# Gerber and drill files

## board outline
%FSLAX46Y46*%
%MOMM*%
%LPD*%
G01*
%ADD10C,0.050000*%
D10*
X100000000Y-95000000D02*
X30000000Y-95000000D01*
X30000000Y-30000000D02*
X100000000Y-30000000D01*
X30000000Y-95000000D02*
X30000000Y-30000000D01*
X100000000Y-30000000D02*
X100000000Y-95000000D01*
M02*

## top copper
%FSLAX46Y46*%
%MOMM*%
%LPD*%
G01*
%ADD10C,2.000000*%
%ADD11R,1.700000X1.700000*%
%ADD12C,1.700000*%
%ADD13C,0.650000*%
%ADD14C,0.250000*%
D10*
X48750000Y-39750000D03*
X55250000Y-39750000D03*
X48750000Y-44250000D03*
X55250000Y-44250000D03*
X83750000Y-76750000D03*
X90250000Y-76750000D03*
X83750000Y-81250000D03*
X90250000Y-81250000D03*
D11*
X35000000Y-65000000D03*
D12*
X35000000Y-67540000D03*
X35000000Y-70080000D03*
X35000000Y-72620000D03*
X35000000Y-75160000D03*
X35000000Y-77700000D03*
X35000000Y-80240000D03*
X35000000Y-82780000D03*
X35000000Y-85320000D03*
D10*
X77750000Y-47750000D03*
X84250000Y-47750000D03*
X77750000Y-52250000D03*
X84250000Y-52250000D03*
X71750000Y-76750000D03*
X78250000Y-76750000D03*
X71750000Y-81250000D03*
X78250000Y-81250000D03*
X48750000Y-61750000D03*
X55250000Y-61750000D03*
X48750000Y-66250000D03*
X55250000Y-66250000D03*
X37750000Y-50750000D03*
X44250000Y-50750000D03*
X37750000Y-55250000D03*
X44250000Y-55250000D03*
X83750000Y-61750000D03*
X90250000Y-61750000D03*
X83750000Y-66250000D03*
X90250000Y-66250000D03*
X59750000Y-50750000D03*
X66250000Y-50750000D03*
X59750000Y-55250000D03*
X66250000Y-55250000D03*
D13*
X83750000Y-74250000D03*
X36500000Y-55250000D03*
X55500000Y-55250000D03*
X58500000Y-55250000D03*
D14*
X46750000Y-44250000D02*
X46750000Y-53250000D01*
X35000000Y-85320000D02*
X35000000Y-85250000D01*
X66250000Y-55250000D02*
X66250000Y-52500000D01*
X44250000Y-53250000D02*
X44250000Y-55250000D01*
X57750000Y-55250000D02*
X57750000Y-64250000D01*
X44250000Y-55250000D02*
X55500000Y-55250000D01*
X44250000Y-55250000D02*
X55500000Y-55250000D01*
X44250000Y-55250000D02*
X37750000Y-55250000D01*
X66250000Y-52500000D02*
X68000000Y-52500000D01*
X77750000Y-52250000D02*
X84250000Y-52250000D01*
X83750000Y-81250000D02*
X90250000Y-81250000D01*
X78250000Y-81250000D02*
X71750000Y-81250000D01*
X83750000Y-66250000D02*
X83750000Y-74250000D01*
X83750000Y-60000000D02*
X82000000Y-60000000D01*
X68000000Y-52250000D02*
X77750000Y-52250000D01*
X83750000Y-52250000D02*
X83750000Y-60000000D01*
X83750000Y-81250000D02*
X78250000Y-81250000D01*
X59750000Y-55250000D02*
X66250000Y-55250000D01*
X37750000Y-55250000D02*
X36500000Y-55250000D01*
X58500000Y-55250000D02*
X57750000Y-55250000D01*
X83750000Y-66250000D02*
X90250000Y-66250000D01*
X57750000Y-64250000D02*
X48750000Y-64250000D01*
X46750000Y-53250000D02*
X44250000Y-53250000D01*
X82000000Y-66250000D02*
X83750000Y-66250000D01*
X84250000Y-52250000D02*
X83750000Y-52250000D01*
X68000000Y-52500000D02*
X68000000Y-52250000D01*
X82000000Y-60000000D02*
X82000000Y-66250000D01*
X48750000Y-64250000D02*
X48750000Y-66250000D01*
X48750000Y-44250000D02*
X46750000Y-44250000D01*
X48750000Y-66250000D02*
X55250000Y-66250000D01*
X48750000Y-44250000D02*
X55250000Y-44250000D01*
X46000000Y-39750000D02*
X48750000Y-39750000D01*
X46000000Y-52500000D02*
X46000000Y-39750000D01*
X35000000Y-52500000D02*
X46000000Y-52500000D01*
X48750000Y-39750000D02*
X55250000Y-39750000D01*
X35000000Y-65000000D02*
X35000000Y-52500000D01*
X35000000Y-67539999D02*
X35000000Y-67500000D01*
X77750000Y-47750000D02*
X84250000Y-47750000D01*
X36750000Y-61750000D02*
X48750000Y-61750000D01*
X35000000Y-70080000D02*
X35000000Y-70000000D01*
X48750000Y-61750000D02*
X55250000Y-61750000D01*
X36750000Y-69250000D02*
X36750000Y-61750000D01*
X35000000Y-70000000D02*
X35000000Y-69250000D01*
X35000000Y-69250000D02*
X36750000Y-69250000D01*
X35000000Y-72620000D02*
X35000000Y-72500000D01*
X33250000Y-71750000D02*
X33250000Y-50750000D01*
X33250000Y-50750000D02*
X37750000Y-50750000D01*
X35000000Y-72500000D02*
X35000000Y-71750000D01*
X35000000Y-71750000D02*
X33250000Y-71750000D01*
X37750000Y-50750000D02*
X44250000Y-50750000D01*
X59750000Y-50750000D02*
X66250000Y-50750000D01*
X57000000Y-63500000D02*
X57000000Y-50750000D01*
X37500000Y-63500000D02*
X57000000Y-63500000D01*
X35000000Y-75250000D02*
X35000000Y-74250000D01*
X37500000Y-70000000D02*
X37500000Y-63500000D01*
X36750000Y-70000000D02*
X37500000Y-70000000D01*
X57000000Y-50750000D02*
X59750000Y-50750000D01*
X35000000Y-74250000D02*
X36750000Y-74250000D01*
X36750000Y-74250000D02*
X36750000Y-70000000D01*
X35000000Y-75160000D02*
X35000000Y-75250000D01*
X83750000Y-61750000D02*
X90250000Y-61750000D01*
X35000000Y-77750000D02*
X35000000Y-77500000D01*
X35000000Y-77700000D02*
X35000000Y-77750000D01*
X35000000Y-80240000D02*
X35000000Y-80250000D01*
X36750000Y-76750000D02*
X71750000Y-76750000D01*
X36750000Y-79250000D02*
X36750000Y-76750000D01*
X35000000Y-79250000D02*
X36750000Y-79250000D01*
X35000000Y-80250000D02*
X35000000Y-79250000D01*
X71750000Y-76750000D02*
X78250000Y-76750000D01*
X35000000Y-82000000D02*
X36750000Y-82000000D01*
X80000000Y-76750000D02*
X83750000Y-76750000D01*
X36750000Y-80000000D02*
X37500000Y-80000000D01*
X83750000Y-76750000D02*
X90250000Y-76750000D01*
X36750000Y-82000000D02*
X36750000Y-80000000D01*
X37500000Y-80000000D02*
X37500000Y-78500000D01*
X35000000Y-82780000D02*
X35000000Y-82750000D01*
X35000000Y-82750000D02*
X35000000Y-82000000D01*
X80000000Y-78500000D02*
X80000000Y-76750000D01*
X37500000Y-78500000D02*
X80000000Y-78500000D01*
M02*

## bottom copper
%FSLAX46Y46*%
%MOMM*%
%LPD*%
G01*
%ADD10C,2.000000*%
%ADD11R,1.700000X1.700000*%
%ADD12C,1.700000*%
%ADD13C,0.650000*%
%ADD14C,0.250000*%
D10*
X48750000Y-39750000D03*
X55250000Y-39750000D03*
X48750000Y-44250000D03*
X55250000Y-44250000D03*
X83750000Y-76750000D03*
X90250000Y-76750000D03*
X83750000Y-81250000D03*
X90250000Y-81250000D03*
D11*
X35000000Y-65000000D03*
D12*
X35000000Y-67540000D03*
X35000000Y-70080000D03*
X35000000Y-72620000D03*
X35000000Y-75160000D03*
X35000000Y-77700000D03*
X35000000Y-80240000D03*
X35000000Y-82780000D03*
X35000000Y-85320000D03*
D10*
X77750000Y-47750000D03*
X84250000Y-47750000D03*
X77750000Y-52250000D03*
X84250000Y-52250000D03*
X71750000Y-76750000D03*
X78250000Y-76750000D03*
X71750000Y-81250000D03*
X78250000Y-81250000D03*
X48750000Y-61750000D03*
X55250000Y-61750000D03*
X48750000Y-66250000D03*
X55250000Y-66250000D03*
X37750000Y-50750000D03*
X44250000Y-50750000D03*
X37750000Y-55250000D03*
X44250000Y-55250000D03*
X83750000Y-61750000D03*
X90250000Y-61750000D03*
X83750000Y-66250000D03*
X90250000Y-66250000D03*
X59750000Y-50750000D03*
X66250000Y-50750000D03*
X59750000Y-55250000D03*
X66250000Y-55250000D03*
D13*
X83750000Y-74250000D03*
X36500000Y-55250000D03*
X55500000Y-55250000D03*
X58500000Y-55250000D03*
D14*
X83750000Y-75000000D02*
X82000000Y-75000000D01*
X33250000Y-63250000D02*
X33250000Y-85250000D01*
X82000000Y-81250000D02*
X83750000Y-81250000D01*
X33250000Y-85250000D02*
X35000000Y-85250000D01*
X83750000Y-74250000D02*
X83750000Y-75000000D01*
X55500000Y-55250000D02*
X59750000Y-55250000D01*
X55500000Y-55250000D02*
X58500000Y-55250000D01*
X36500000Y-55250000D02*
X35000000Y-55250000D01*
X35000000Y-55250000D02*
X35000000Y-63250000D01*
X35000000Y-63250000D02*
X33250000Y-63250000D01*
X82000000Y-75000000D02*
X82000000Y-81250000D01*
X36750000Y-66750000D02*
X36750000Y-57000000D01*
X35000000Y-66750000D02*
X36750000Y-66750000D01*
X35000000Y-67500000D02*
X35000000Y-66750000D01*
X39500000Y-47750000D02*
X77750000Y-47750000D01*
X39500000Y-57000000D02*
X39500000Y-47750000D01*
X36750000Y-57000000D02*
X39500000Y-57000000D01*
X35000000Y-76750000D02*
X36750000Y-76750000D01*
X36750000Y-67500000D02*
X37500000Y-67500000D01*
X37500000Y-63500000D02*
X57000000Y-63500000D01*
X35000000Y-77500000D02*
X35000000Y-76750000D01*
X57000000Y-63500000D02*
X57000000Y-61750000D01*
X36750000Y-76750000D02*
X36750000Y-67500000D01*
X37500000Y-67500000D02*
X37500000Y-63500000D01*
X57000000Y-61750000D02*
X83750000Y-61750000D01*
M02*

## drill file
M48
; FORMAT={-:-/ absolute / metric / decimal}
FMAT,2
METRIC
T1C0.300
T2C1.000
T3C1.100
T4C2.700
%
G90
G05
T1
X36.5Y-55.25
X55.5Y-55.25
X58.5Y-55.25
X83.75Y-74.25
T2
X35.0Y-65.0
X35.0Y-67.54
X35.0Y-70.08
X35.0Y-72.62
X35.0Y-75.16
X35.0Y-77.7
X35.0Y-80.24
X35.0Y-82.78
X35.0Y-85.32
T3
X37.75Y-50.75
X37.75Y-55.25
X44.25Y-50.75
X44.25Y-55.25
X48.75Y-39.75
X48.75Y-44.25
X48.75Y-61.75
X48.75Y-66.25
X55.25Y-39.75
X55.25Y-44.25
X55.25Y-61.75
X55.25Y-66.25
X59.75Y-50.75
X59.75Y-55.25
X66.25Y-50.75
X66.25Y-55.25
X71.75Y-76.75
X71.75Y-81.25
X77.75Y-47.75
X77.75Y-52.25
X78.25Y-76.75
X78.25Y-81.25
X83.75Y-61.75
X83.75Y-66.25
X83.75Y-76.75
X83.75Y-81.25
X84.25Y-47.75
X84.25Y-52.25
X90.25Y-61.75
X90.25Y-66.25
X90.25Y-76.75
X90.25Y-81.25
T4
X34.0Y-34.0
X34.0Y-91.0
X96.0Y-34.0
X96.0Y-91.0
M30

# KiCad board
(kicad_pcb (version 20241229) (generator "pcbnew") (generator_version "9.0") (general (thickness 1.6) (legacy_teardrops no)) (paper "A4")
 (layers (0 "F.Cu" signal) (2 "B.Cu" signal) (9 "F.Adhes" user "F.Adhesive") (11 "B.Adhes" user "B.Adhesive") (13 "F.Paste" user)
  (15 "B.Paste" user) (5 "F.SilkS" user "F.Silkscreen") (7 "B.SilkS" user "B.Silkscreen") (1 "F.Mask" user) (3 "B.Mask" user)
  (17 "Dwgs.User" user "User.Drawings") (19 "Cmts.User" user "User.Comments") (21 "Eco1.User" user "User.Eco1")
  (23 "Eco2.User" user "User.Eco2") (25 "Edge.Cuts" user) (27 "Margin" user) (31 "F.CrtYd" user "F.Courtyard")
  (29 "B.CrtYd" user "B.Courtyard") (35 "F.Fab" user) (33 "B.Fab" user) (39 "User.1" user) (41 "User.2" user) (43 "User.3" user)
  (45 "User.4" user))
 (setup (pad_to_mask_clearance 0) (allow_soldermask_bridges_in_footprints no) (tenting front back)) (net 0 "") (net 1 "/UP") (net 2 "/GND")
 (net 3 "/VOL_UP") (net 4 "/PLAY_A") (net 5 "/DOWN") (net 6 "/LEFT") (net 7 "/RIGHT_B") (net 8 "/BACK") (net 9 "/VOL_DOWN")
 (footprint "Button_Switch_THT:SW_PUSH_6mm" (layer "F.Cu") (at 48.75 39.75)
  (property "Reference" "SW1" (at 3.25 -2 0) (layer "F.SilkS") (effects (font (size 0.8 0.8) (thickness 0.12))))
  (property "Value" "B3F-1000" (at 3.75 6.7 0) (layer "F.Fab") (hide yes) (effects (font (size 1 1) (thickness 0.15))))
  (pad "1" thru_hole circle (at 0 0 90) (size 2 2) (drill 1.1) (layers "*.Cu" "*.Mask") (remove_unused_layers no) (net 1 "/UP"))
  (pad "1" thru_hole circle (at 6.5 0 90) (size 2 2) (drill 1.1) (layers "*.Cu" "*.Mask") (remove_unused_layers no) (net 1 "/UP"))
  (pad "2" thru_hole circle (at 0 4.5 90) (size 2 2) (drill 1.1) (layers "*.Cu" "*.Mask") (remove_unused_layers no) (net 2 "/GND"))
  (pad "2" thru_hole circle (at 6.5 4.5 90) (size 2 2) (drill 1.1) (layers "*.Cu" "*.Mask") (remove_unused_layers no) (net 2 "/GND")))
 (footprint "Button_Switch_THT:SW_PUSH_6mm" (layer "F.Cu") (at 83.75 76.75)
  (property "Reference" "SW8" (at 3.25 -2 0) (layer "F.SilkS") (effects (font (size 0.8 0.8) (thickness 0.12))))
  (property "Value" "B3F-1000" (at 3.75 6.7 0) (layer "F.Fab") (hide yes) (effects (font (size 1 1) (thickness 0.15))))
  (pad "1" thru_hole circle (at 0 0 90) (size 2 2) (drill 1.1) (layers "*.Cu" "*.Mask") (remove_unused_layers no) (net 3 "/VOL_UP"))
  (pad "1" thru_hole circle (at 6.5 0 90) (size 2 2) (drill 1.1) (layers "*.Cu" "*.Mask") (remove_unused_layers no) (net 3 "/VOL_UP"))
  (pad "2" thru_hole circle (at 0 4.5 90) (size 2 2) (drill 1.1) (layers "*.Cu" "*.Mask") (remove_unused_layers no) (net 2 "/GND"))
  (pad "2" thru_hole circle (at 6.5 4.5 90) (size 2 2) (drill 1.1) (layers "*.Cu" "*.Mask") (remove_unused_layers no) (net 2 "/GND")))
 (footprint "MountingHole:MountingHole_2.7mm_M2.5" (layer "F.Cu") (at 34 91)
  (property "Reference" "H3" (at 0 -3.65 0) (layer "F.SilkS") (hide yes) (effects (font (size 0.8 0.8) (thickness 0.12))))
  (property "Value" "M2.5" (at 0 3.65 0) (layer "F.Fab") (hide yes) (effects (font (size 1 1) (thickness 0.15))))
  (pad "" np_thru_hole circle (at 0 0) (size 2.7 2.7) (drill 2.7) (layers "*.Cu" "*.Mask")))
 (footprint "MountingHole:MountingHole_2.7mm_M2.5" (layer "F.Cu") (at 96 91)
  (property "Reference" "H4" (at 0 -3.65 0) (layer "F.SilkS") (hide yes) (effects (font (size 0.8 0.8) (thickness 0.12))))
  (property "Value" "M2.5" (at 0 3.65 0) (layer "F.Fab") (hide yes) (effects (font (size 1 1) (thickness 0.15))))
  (pad "" np_thru_hole circle (at 0 0) (size 2.7 2.7) (drill 2.7) (layers "*.Cu" "*.Mask")))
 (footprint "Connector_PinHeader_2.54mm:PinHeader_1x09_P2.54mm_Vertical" (layer "F.Cu") (at 35 65)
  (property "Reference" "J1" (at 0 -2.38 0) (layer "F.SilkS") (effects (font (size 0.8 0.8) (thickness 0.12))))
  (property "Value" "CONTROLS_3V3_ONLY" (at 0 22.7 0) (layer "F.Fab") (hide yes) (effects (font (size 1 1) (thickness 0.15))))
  (pad "1" thru_hole rect (at 0 0) (size 1.7 1.7) (drill 1) (layers "*.Cu" "*.Mask") (remove_unused_layers no) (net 1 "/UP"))
  (pad "2" thru_hole circle (at 0 2.54) (size 1.7 1.7) (drill 1) (layers "*.Cu" "*.Mask") (remove_unused_layers no) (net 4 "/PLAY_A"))
  (pad "3" thru_hole circle (at 0 5.08) (size 1.7 1.7) (drill 1) (layers "*.Cu" "*.Mask") (remove_unused_layers no) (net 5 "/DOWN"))
  (pad "4" thru_hole circle (at 0 7.62) (size 1.7 1.7) (drill 1) (layers "*.Cu" "*.Mask") (remove_unused_layers no) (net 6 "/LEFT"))
  (pad "5" thru_hole circle (at 0 10.16) (size 1.7 1.7) (drill 1) (layers "*.Cu" "*.Mask") (remove_unused_layers no) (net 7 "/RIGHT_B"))
  (pad "6" thru_hole circle (at 0 12.7) (size 1.7 1.7) (drill 1) (layers "*.Cu" "*.Mask") (remove_unused_layers no) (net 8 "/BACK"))
  (pad "7" thru_hole circle (at 0 15.24) (size 1.7 1.7) (drill 1) (layers "*.Cu" "*.Mask") (remove_unused_layers no) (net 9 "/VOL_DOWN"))
  (pad "8" thru_hole circle (at 0 17.78) (size 1.7 1.7) (drill 1) (layers "*.Cu" "*.Mask") (remove_unused_layers no) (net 3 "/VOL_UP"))
  (pad "9" thru_hole circle (at 0 20.32) (size 1.7 1.7) (drill 1) (layers "*.Cu" "*.Mask") (remove_unused_layers no) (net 2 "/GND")))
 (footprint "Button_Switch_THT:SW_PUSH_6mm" (layer "F.Cu") (at 77.75 47.75)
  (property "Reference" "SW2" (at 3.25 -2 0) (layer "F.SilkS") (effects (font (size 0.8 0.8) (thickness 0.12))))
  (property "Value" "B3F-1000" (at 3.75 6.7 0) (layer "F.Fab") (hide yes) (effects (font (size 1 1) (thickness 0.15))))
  (pad "1" thru_hole circle (at 0 0 90) (size 2 2) (drill 1.1) (layers "*.Cu" "*.Mask") (remove_unused_layers no) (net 4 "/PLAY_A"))
  (pad "1" thru_hole circle (at 6.5 0 90) (size 2 2) (drill 1.1) (layers "*.Cu" "*.Mask") (remove_unused_layers no) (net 4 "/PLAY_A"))
  (pad "2" thru_hole circle (at 0 4.5 90) (size 2 2) (drill 1.1) (layers "*.Cu" "*.Mask") (remove_unused_layers no) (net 2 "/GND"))
  (pad "2" thru_hole circle (at 6.5 4.5 90) (size 2 2) (drill 1.1) (layers "*.Cu" "*.Mask") (remove_unused_layers no) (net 2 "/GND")))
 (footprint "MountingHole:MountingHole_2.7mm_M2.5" (layer "F.Cu") (at 34 34)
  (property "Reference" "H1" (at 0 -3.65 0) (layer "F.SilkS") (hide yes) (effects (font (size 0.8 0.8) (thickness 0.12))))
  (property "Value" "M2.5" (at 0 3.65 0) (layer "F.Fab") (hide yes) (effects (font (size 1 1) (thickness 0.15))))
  (pad "" np_thru_hole circle (at 0 0) (size 2.7 2.7) (drill 2.7) (layers "*.Cu" "*.Mask")))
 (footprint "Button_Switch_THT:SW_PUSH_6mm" (layer "F.Cu") (at 71.75 76.75)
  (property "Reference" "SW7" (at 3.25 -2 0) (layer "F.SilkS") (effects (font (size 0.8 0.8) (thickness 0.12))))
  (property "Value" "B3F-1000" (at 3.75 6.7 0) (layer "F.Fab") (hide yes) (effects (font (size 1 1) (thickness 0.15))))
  (pad "1" thru_hole circle (at 0 0 90) (size 2 2) (drill 1.1) (layers "*.Cu" "*.Mask") (remove_unused_layers no) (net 9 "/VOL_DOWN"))
  (pad "1" thru_hole circle (at 6.5 0 90) (size 2 2) (drill 1.1) (layers "*.Cu" "*.Mask") (remove_unused_layers no) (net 9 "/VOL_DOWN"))
  (pad "2" thru_hole circle (at 0 4.5 90) (size 2 2) (drill 1.1) (layers "*.Cu" "*.Mask") (remove_unused_layers no) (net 2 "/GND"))
  (pad "2" thru_hole circle (at 6.5 4.5 90) (size 2 2) (drill 1.1) (layers "*.Cu" "*.Mask") (remove_unused_layers no) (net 2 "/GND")))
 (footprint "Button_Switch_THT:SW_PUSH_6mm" (layer "F.Cu") (at 48.75 61.75)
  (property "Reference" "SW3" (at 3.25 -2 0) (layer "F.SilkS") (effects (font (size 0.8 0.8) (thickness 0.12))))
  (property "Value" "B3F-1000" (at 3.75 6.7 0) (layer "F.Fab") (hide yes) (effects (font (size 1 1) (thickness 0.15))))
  (pad "1" thru_hole circle (at 0 0 90) (size 2 2) (drill 1.1) (layers "*.Cu" "*.Mask") (remove_unused_layers no) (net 5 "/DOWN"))
  (pad "1" thru_hole circle (at 6.5 0 90) (size 2 2) (drill 1.1) (layers "*.Cu" "*.Mask") (remove_unused_layers no) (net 5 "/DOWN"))
  (pad "2" thru_hole circle (at 0 4.5 90) (size 2 2) (drill 1.1) (layers "*.Cu" "*.Mask") (remove_unused_layers no) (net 2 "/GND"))
  (pad "2" thru_hole circle (at 6.5 4.5 90) (size 2 2) (drill 1.1) (layers "*.Cu" "*.Mask") (remove_unused_layers no) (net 2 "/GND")))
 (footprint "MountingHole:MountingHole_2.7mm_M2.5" (layer "F.Cu") (at 96 34)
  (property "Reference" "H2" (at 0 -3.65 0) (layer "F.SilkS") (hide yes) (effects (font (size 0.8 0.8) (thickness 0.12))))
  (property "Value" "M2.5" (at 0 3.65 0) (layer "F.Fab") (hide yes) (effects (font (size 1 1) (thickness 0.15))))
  (pad "" np_thru_hole circle (at 0 0) (size 2.7 2.7) (drill 2.7) (layers "*.Cu" "*.Mask")))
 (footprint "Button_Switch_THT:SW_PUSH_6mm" (layer "F.Cu") (at 37.75 50.75)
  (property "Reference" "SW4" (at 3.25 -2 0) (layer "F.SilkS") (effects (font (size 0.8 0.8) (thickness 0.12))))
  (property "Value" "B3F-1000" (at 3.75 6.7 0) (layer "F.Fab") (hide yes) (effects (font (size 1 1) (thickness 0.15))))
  (pad "1" thru_hole circle (at 0 0 90) (size 2 2) (drill 1.1) (layers "*.Cu" "*.Mask") (remove_unused_layers no) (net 6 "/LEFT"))
  (pad "1" thru_hole circle (at 6.5 0 90) (size 2 2) (drill 1.1) (layers "*.Cu" "*.Mask") (remove_unused_layers no) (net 6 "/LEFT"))
  (pad "2" thru_hole circle (at 0 4.5 90) (size 2 2) (drill 1.1) (layers "*.Cu" "*.Mask") (remove_unused_layers no) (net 2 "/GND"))
  (pad "2" thru_hole circle (at 6.5 4.5 90) (size 2 2) (drill 1.1) (layers "*.Cu" "*.Mask") (remove_unused_layers no) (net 2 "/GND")))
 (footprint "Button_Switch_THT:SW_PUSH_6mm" (layer "F.Cu") (at 83.75 61.75)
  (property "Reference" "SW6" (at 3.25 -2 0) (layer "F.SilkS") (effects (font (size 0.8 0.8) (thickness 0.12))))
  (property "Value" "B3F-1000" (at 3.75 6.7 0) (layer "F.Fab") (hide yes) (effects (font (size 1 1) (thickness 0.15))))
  (pad "1" thru_hole circle (at 0 0 90) (size 2 2) (drill 1.1) (layers "*.Cu" "*.Mask") (remove_unused_layers no) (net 8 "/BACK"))
  (pad "1" thru_hole circle (at 6.5 0 90) (size 2 2) (drill 1.1) (layers "*.Cu" "*.Mask") (remove_unused_layers no) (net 8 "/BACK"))
  (pad "2" thru_hole circle (at 0 4.5 90) (size 2 2) (drill 1.1) (layers "*.Cu" "*.Mask") (remove_unused_layers no) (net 2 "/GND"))
  (pad "2" thru_hole circle (at 6.5 4.5 90) (size 2 2) (drill 1.1) (layers "*.Cu" "*.Mask") (remove_unused_layers no) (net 2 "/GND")))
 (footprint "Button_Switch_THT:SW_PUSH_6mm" (layer "F.Cu") (at 59.75 50.75)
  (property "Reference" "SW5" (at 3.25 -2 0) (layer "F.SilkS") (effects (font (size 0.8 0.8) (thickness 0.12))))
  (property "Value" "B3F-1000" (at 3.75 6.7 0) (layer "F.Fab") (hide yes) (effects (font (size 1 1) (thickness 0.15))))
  (pad "1" thru_hole circle (at 0 0 90) (size 2 2) (drill 1.1) (layers "*.Cu" "*.Mask") (remove_unused_layers no) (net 7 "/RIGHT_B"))
  (pad "1" thru_hole circle (at 6.5 0 90) (size 2 2) (drill 1.1) (layers "*.Cu" "*.Mask") (remove_unused_layers no) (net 7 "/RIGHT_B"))
  (pad "2" thru_hole circle (at 0 4.5 90) (size 2 2) (drill 1.1) (layers "*.Cu" "*.Mask") (remove_unused_layers no) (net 2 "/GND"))
  (pad "2" thru_hole circle (at 6.5 4.5 90) (size 2 2) (drill 1.1) (layers "*.Cu" "*.Mask") (remove_unused_layers no) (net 2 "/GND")))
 (gr_line (start 100 95) (end 30 95) (stroke (width 0.05) (type default)) (layer "Edge.Cuts"))
 (gr_line (start 30 30) (end 100 30) (stroke (width 0.05) (type default)) (layer "Edge.Cuts"))
 (gr_line (start 30 95) (end 30 30) (stroke (width 0.05) (type default)) (layer "Edge.Cuts"))
 (gr_line (start 100 30) (end 100 95) (stroke (width 0.05) (type default)) (layer "Edge.Cuts"))
 (segment (start 46.75 44.25) (end 46.75 53.25) (width 0.25) (layer "F.Cu") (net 2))
 (segment (start 35 85.32) (end 35 85.25) (width 0.25) (layer "F.Cu") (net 2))
 (segment (start 66.25 55.25) (end 66.25 52.5) (width 0.25) (layer "F.Cu") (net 2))
 (segment (start 44.25 53.25) (end 44.25 55.25) (width 0.25) (layer "F.Cu") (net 2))
 (segment (start 57.75 55.25) (end 57.75 64.25) (width 0.25) (layer "F.Cu") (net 2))
 (segment (start 44.25 55.25) (end 55.5 55.25) (width 0.25) (layer "F.Cu") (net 2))
 (segment (start 44.25 55.25) (end 55.5 55.25) (width 0.25) (layer "F.Cu") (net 2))
 (segment (start 44.25 55.25) (end 37.75 55.25) (width 0.25) (layer "F.Cu") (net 2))
 (segment (start 66.25 52.5) (end 68 52.5) (width 0.25) (layer "F.Cu") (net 2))
 (segment (start 77.75 52.25) (end 84.25 52.25) (width 0.25) (layer "F.Cu") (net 2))
 (segment (start 83.75 81.25) (end 90.25 81.25) (width 0.25) (layer "F.Cu") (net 2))
 (segment (start 78.25 81.25) (end 71.75 81.25) (width 0.25) (layer "F.Cu") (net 2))
 (segment (start 83.75 66.25) (end 83.75 74.25) (width 0.25) (layer "F.Cu") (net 2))
 (segment (start 83.75 60) (end 82 60) (width 0.25) (layer "F.Cu") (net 2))
 (segment (start 68 52.25) (end 77.75 52.25) (width 0.25) (layer "F.Cu") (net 2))
 (segment (start 83.75 52.25) (end 83.75 60) (width 0.25) (layer "F.Cu") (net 2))
 (segment (start 83.75 81.25) (end 78.25 81.25) (width 0.25) (layer "F.Cu") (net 2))
 (segment (start 59.75 55.25) (end 66.25 55.25) (width 0.25) (layer "F.Cu") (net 2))
 (segment (start 37.75 55.25) (end 36.5 55.25) (width 0.25) (layer "F.Cu") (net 2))
 (segment (start 58.5 55.25) (end 57.75 55.25) (width 0.25) (layer "F.Cu") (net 2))
 (segment (start 83.75 66.25) (end 90.25 66.25) (width 0.25) (layer "F.Cu") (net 2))
 (segment (start 57.75 64.25) (end 48.75 64.25) (width 0.25) (layer "F.Cu") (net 2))
 (segment (start 46.75 53.25) (end 44.25 53.25) (width 0.25) (layer "F.Cu") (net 2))
 (segment (start 82 66.25) (end 83.75 66.25) (width 0.25) (layer "F.Cu") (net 2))
 (segment (start 84.25 52.25) (end 83.75 52.25) (width 0.25) (layer "F.Cu") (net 2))
 (segment (start 68 52.5) (end 68 52.25) (width 0.25) (layer "F.Cu") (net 2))
 (segment (start 82 60) (end 82 66.25) (width 0.25) (layer "F.Cu") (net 2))
 (segment (start 48.75 64.25) (end 48.75 66.25) (width 0.25) (layer "F.Cu") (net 2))
 (segment (start 48.75 44.25) (end 46.75 44.25) (width 0.25) (layer "F.Cu") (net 2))
 (segment (start 48.75 66.25) (end 55.25 66.25) (width 0.25) (layer "F.Cu") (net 2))
 (segment (start 48.75 44.25) (end 55.25 44.25) (width 0.25) (layer "F.Cu") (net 2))
 (via (at 83.75 74.25) (size 0.65) (drill 0.3) (layers "F.Cu" "B.Cu") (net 2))
 (via (at 36.5 55.25) (size 0.65) (drill 0.3) (layers "F.Cu" "B.Cu") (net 2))
 (via (at 55.5 55.25) (size 0.65) (drill 0.3) (layers "F.Cu" "B.Cu") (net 2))
 (via (at 58.5 55.25) (size 0.65) (drill 0.3) (layers "F.Cu" "B.Cu") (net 2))
 (segment (start 83.75 75) (end 82 75) (width 0.25) (layer "B.Cu") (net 2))
 (segment (start 33.25 63.25) (end 33.25 85.25) (width 0.25) (layer "B.Cu") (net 2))
 (segment (start 82 81.25) (end 83.75 81.25) (width 0.25) (layer "B.Cu") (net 2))
 (segment (start 33.25 85.25) (end 35 85.25) (width 0.25) (layer "B.Cu") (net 2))
 (segment (start 83.75 74.25) (end 83.75 75) (width 0.25) (layer "B.Cu") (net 2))
 (segment (start 55.5 55.25) (end 59.75 55.25) (width 0.25) (layer "B.Cu") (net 2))
 (segment (start 55.5 55.25) (end 58.5 55.25) (width 0.25) (layer "B.Cu") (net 2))
 (segment (start 36.5 55.25) (end 35 55.25) (width 0.25) (layer "B.Cu") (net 2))
 (segment (start 35 55.25) (end 35 63.25) (width 0.25) (layer "B.Cu") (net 2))
 (segment (start 35 63.25) (end 33.25 63.25) (width 0.25) (layer "B.Cu") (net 2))
 (segment (start 82 75) (end 82 81.25) (width 0.25) (layer "B.Cu") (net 2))
 (segment (start 46 39.75) (end 48.75 39.75) (width 0.25) (layer "F.Cu") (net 1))
 (segment (start 46 52.5) (end 46 39.75) (width 0.25) (layer "F.Cu") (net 1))
 (segment (start 35 52.5) (end 46 52.5) (width 0.25) (layer "F.Cu") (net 1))
 (segment (start 48.75 39.75) (end 55.25 39.75) (width 0.25) (layer "F.Cu") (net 1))
 (segment (start 35 65) (end 35 52.5) (width 0.25) (layer "F.Cu") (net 1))
 (segment (start 35 67.539999) (end 35 67.5) (width 0.25) (layer "F.Cu") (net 4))
 (segment (start 77.75 47.75) (end 84.25 47.75) (width 0.25) (layer "F.Cu") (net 4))
 (segment (start 36.75 66.75) (end 36.75 57) (width 0.25) (layer "B.Cu") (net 4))
 (segment (start 35 66.75) (end 36.75 66.75) (width 0.25) (layer "B.Cu") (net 4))
 (segment (start 35 67.5) (end 35 66.75) (width 0.25) (layer "B.Cu") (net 4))
 (segment (start 39.5 47.75) (end 77.75 47.75) (width 0.25) (layer "B.Cu") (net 4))
 (segment (start 39.5 57) (end 39.5 47.75) (width 0.25) (layer "B.Cu") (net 4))
 (segment (start 36.75 57) (end 39.5 57) (width 0.25) (layer "B.Cu") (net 4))
 (segment (start 36.75 61.75) (end 48.75 61.75) (width 0.25) (layer "F.Cu") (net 5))
 (segment (start 35 70.08) (end 35 70) (width 0.25) (layer "F.Cu") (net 5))
 (segment (start 48.75 61.75) (end 55.25 61.75) (width 0.25) (layer "F.Cu") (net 5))
 (segment (start 36.75 69.25) (end 36.75 61.75) (width 0.25) (layer "F.Cu") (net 5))
 (segment (start 35 70) (end 35 69.25) (width 0.25) (layer "F.Cu") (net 5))
 (segment (start 35 69.25) (end 36.75 69.25) (width 0.25) (layer "F.Cu") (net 5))
 (segment (start 35 72.62) (end 35 72.5) (width 0.25) (layer "F.Cu") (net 6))
 (segment (start 33.25 71.75) (end 33.25 50.75) (width 0.25) (layer "F.Cu") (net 6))
 (segment (start 33.25 50.75) (end 37.75 50.75) (width 0.25) (layer "F.Cu") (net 6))
 (segment (start 35 72.5) (end 35 71.75) (width 0.25) (layer "F.Cu") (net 6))
 (segment (start 35 71.75) (end 33.25 71.75) (width 0.25) (layer "F.Cu") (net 6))
 (segment (start 37.75 50.75) (end 44.25 50.75) (width 0.25) (layer "F.Cu") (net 6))
 (segment (start 59.75 50.75) (end 66.25 50.75) (width 0.25) (layer "F.Cu") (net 7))
 (segment (start 57 63.5) (end 57 50.75) (width 0.25) (layer "F.Cu") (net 7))
 (segment (start 37.5 63.5) (end 57 63.5) (width 0.25) (layer "F.Cu") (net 7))
 (segment (start 35 75.25) (end 35 74.25) (width 0.25) (layer "F.Cu") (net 7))
 (segment (start 37.5 70) (end 37.5 63.5) (width 0.25) (layer "F.Cu") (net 7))
 (segment (start 36.75 70) (end 37.5 70) (width 0.25) (layer "F.Cu") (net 7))
 (segment (start 57 50.75) (end 59.75 50.75) (width 0.25) (layer "F.Cu") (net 7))
 (segment (start 35 74.25) (end 36.75 74.25) (width 0.25) (layer "F.Cu") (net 7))
 (segment (start 36.75 74.25) (end 36.75 70) (width 0.25) (layer "F.Cu") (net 7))
 (segment (start 35 75.16) (end 35 75.25) (width 0.25) (layer "F.Cu") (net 7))
 (segment (start 83.75 61.75) (end 90.25 61.75) (width 0.25) (layer "F.Cu") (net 8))
 (segment (start 35 77.75) (end 35 77.5) (width 0.25) (layer "F.Cu") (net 8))
 (segment (start 35 77.7) (end 35 77.75) (width 0.25) (layer "F.Cu") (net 8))
 (segment (start 35 76.75) (end 36.75 76.75) (width 0.25) (layer "B.Cu") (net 8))
 (segment (start 36.75 67.5) (end 37.5 67.5) (width 0.25) (layer "B.Cu") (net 8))
 (segment (start 37.5 63.5) (end 57 63.5) (width 0.25) (layer "B.Cu") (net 8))
 (segment (start 35 77.5) (end 35 76.75) (width 0.25) (layer "B.Cu") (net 8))
 (segment (start 57 63.5) (end 57 61.75) (width 0.25) (layer "B.Cu") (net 8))
 (segment (start 36.75 76.75) (end 36.75 67.5) (width 0.25) (layer "B.Cu") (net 8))
 (segment (start 37.5 67.5) (end 37.5 63.5) (width 0.25) (layer "B.Cu") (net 8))
 (segment (start 57 61.75) (end 83.75 61.75) (width 0.25) (layer "B.Cu") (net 8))
 (segment (start 35 80.24) (end 35 80.25) (width 0.25) (layer "F.Cu") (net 9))
 (segment (start 36.75 76.75) (end 71.75 76.75) (width 0.25) (layer "F.Cu") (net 9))
 (segment (start 36.75 79.25) (end 36.75 76.75) (width 0.25) (layer "F.Cu") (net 9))
 (segment (start 35 79.25) (end 36.75 79.25) (width 0.25) (layer "F.Cu") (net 9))
 (segment (start 35 80.25) (end 35 79.25) (width 0.25) (layer "F.Cu") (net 9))
 (segment (start 71.75 76.75) (end 78.25 76.75) (width 0.25) (layer "F.Cu") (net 9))
 (segment (start 35 82) (end 36.75 82) (width 0.25) (layer "F.Cu") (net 3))
 (segment (start 80 76.75) (end 83.75 76.75) (width 0.25) (layer "F.Cu") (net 3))
 (segment (start 36.75 80) (end 37.5 80) (width 0.25) (layer "F.Cu") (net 3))
 (segment (start 83.75 76.75) (end 90.25 76.75) (width 0.25) (layer "F.Cu") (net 3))
 (segment (start 36.75 82) (end 36.75 80) (width 0.25) (layer "F.Cu") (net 3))
 (segment (start 37.5 80) (end 37.5 78.5) (width 0.25) (layer "F.Cu") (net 3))
 (segment (start 35 82.78) (end 35 82.75) (width 0.25) (layer "F.Cu") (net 3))
 (segment (start 35 82.75) (end 35 82) (width 0.25) (layer "F.Cu") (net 3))
 (segment (start 80 78.5) (end 80 76.75) (width 0.25) (layer "F.Cu") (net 3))
 (segment (start 37.5 78.5) (end 80 78.5) (width 0.25) (layer "F.Cu") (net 3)))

